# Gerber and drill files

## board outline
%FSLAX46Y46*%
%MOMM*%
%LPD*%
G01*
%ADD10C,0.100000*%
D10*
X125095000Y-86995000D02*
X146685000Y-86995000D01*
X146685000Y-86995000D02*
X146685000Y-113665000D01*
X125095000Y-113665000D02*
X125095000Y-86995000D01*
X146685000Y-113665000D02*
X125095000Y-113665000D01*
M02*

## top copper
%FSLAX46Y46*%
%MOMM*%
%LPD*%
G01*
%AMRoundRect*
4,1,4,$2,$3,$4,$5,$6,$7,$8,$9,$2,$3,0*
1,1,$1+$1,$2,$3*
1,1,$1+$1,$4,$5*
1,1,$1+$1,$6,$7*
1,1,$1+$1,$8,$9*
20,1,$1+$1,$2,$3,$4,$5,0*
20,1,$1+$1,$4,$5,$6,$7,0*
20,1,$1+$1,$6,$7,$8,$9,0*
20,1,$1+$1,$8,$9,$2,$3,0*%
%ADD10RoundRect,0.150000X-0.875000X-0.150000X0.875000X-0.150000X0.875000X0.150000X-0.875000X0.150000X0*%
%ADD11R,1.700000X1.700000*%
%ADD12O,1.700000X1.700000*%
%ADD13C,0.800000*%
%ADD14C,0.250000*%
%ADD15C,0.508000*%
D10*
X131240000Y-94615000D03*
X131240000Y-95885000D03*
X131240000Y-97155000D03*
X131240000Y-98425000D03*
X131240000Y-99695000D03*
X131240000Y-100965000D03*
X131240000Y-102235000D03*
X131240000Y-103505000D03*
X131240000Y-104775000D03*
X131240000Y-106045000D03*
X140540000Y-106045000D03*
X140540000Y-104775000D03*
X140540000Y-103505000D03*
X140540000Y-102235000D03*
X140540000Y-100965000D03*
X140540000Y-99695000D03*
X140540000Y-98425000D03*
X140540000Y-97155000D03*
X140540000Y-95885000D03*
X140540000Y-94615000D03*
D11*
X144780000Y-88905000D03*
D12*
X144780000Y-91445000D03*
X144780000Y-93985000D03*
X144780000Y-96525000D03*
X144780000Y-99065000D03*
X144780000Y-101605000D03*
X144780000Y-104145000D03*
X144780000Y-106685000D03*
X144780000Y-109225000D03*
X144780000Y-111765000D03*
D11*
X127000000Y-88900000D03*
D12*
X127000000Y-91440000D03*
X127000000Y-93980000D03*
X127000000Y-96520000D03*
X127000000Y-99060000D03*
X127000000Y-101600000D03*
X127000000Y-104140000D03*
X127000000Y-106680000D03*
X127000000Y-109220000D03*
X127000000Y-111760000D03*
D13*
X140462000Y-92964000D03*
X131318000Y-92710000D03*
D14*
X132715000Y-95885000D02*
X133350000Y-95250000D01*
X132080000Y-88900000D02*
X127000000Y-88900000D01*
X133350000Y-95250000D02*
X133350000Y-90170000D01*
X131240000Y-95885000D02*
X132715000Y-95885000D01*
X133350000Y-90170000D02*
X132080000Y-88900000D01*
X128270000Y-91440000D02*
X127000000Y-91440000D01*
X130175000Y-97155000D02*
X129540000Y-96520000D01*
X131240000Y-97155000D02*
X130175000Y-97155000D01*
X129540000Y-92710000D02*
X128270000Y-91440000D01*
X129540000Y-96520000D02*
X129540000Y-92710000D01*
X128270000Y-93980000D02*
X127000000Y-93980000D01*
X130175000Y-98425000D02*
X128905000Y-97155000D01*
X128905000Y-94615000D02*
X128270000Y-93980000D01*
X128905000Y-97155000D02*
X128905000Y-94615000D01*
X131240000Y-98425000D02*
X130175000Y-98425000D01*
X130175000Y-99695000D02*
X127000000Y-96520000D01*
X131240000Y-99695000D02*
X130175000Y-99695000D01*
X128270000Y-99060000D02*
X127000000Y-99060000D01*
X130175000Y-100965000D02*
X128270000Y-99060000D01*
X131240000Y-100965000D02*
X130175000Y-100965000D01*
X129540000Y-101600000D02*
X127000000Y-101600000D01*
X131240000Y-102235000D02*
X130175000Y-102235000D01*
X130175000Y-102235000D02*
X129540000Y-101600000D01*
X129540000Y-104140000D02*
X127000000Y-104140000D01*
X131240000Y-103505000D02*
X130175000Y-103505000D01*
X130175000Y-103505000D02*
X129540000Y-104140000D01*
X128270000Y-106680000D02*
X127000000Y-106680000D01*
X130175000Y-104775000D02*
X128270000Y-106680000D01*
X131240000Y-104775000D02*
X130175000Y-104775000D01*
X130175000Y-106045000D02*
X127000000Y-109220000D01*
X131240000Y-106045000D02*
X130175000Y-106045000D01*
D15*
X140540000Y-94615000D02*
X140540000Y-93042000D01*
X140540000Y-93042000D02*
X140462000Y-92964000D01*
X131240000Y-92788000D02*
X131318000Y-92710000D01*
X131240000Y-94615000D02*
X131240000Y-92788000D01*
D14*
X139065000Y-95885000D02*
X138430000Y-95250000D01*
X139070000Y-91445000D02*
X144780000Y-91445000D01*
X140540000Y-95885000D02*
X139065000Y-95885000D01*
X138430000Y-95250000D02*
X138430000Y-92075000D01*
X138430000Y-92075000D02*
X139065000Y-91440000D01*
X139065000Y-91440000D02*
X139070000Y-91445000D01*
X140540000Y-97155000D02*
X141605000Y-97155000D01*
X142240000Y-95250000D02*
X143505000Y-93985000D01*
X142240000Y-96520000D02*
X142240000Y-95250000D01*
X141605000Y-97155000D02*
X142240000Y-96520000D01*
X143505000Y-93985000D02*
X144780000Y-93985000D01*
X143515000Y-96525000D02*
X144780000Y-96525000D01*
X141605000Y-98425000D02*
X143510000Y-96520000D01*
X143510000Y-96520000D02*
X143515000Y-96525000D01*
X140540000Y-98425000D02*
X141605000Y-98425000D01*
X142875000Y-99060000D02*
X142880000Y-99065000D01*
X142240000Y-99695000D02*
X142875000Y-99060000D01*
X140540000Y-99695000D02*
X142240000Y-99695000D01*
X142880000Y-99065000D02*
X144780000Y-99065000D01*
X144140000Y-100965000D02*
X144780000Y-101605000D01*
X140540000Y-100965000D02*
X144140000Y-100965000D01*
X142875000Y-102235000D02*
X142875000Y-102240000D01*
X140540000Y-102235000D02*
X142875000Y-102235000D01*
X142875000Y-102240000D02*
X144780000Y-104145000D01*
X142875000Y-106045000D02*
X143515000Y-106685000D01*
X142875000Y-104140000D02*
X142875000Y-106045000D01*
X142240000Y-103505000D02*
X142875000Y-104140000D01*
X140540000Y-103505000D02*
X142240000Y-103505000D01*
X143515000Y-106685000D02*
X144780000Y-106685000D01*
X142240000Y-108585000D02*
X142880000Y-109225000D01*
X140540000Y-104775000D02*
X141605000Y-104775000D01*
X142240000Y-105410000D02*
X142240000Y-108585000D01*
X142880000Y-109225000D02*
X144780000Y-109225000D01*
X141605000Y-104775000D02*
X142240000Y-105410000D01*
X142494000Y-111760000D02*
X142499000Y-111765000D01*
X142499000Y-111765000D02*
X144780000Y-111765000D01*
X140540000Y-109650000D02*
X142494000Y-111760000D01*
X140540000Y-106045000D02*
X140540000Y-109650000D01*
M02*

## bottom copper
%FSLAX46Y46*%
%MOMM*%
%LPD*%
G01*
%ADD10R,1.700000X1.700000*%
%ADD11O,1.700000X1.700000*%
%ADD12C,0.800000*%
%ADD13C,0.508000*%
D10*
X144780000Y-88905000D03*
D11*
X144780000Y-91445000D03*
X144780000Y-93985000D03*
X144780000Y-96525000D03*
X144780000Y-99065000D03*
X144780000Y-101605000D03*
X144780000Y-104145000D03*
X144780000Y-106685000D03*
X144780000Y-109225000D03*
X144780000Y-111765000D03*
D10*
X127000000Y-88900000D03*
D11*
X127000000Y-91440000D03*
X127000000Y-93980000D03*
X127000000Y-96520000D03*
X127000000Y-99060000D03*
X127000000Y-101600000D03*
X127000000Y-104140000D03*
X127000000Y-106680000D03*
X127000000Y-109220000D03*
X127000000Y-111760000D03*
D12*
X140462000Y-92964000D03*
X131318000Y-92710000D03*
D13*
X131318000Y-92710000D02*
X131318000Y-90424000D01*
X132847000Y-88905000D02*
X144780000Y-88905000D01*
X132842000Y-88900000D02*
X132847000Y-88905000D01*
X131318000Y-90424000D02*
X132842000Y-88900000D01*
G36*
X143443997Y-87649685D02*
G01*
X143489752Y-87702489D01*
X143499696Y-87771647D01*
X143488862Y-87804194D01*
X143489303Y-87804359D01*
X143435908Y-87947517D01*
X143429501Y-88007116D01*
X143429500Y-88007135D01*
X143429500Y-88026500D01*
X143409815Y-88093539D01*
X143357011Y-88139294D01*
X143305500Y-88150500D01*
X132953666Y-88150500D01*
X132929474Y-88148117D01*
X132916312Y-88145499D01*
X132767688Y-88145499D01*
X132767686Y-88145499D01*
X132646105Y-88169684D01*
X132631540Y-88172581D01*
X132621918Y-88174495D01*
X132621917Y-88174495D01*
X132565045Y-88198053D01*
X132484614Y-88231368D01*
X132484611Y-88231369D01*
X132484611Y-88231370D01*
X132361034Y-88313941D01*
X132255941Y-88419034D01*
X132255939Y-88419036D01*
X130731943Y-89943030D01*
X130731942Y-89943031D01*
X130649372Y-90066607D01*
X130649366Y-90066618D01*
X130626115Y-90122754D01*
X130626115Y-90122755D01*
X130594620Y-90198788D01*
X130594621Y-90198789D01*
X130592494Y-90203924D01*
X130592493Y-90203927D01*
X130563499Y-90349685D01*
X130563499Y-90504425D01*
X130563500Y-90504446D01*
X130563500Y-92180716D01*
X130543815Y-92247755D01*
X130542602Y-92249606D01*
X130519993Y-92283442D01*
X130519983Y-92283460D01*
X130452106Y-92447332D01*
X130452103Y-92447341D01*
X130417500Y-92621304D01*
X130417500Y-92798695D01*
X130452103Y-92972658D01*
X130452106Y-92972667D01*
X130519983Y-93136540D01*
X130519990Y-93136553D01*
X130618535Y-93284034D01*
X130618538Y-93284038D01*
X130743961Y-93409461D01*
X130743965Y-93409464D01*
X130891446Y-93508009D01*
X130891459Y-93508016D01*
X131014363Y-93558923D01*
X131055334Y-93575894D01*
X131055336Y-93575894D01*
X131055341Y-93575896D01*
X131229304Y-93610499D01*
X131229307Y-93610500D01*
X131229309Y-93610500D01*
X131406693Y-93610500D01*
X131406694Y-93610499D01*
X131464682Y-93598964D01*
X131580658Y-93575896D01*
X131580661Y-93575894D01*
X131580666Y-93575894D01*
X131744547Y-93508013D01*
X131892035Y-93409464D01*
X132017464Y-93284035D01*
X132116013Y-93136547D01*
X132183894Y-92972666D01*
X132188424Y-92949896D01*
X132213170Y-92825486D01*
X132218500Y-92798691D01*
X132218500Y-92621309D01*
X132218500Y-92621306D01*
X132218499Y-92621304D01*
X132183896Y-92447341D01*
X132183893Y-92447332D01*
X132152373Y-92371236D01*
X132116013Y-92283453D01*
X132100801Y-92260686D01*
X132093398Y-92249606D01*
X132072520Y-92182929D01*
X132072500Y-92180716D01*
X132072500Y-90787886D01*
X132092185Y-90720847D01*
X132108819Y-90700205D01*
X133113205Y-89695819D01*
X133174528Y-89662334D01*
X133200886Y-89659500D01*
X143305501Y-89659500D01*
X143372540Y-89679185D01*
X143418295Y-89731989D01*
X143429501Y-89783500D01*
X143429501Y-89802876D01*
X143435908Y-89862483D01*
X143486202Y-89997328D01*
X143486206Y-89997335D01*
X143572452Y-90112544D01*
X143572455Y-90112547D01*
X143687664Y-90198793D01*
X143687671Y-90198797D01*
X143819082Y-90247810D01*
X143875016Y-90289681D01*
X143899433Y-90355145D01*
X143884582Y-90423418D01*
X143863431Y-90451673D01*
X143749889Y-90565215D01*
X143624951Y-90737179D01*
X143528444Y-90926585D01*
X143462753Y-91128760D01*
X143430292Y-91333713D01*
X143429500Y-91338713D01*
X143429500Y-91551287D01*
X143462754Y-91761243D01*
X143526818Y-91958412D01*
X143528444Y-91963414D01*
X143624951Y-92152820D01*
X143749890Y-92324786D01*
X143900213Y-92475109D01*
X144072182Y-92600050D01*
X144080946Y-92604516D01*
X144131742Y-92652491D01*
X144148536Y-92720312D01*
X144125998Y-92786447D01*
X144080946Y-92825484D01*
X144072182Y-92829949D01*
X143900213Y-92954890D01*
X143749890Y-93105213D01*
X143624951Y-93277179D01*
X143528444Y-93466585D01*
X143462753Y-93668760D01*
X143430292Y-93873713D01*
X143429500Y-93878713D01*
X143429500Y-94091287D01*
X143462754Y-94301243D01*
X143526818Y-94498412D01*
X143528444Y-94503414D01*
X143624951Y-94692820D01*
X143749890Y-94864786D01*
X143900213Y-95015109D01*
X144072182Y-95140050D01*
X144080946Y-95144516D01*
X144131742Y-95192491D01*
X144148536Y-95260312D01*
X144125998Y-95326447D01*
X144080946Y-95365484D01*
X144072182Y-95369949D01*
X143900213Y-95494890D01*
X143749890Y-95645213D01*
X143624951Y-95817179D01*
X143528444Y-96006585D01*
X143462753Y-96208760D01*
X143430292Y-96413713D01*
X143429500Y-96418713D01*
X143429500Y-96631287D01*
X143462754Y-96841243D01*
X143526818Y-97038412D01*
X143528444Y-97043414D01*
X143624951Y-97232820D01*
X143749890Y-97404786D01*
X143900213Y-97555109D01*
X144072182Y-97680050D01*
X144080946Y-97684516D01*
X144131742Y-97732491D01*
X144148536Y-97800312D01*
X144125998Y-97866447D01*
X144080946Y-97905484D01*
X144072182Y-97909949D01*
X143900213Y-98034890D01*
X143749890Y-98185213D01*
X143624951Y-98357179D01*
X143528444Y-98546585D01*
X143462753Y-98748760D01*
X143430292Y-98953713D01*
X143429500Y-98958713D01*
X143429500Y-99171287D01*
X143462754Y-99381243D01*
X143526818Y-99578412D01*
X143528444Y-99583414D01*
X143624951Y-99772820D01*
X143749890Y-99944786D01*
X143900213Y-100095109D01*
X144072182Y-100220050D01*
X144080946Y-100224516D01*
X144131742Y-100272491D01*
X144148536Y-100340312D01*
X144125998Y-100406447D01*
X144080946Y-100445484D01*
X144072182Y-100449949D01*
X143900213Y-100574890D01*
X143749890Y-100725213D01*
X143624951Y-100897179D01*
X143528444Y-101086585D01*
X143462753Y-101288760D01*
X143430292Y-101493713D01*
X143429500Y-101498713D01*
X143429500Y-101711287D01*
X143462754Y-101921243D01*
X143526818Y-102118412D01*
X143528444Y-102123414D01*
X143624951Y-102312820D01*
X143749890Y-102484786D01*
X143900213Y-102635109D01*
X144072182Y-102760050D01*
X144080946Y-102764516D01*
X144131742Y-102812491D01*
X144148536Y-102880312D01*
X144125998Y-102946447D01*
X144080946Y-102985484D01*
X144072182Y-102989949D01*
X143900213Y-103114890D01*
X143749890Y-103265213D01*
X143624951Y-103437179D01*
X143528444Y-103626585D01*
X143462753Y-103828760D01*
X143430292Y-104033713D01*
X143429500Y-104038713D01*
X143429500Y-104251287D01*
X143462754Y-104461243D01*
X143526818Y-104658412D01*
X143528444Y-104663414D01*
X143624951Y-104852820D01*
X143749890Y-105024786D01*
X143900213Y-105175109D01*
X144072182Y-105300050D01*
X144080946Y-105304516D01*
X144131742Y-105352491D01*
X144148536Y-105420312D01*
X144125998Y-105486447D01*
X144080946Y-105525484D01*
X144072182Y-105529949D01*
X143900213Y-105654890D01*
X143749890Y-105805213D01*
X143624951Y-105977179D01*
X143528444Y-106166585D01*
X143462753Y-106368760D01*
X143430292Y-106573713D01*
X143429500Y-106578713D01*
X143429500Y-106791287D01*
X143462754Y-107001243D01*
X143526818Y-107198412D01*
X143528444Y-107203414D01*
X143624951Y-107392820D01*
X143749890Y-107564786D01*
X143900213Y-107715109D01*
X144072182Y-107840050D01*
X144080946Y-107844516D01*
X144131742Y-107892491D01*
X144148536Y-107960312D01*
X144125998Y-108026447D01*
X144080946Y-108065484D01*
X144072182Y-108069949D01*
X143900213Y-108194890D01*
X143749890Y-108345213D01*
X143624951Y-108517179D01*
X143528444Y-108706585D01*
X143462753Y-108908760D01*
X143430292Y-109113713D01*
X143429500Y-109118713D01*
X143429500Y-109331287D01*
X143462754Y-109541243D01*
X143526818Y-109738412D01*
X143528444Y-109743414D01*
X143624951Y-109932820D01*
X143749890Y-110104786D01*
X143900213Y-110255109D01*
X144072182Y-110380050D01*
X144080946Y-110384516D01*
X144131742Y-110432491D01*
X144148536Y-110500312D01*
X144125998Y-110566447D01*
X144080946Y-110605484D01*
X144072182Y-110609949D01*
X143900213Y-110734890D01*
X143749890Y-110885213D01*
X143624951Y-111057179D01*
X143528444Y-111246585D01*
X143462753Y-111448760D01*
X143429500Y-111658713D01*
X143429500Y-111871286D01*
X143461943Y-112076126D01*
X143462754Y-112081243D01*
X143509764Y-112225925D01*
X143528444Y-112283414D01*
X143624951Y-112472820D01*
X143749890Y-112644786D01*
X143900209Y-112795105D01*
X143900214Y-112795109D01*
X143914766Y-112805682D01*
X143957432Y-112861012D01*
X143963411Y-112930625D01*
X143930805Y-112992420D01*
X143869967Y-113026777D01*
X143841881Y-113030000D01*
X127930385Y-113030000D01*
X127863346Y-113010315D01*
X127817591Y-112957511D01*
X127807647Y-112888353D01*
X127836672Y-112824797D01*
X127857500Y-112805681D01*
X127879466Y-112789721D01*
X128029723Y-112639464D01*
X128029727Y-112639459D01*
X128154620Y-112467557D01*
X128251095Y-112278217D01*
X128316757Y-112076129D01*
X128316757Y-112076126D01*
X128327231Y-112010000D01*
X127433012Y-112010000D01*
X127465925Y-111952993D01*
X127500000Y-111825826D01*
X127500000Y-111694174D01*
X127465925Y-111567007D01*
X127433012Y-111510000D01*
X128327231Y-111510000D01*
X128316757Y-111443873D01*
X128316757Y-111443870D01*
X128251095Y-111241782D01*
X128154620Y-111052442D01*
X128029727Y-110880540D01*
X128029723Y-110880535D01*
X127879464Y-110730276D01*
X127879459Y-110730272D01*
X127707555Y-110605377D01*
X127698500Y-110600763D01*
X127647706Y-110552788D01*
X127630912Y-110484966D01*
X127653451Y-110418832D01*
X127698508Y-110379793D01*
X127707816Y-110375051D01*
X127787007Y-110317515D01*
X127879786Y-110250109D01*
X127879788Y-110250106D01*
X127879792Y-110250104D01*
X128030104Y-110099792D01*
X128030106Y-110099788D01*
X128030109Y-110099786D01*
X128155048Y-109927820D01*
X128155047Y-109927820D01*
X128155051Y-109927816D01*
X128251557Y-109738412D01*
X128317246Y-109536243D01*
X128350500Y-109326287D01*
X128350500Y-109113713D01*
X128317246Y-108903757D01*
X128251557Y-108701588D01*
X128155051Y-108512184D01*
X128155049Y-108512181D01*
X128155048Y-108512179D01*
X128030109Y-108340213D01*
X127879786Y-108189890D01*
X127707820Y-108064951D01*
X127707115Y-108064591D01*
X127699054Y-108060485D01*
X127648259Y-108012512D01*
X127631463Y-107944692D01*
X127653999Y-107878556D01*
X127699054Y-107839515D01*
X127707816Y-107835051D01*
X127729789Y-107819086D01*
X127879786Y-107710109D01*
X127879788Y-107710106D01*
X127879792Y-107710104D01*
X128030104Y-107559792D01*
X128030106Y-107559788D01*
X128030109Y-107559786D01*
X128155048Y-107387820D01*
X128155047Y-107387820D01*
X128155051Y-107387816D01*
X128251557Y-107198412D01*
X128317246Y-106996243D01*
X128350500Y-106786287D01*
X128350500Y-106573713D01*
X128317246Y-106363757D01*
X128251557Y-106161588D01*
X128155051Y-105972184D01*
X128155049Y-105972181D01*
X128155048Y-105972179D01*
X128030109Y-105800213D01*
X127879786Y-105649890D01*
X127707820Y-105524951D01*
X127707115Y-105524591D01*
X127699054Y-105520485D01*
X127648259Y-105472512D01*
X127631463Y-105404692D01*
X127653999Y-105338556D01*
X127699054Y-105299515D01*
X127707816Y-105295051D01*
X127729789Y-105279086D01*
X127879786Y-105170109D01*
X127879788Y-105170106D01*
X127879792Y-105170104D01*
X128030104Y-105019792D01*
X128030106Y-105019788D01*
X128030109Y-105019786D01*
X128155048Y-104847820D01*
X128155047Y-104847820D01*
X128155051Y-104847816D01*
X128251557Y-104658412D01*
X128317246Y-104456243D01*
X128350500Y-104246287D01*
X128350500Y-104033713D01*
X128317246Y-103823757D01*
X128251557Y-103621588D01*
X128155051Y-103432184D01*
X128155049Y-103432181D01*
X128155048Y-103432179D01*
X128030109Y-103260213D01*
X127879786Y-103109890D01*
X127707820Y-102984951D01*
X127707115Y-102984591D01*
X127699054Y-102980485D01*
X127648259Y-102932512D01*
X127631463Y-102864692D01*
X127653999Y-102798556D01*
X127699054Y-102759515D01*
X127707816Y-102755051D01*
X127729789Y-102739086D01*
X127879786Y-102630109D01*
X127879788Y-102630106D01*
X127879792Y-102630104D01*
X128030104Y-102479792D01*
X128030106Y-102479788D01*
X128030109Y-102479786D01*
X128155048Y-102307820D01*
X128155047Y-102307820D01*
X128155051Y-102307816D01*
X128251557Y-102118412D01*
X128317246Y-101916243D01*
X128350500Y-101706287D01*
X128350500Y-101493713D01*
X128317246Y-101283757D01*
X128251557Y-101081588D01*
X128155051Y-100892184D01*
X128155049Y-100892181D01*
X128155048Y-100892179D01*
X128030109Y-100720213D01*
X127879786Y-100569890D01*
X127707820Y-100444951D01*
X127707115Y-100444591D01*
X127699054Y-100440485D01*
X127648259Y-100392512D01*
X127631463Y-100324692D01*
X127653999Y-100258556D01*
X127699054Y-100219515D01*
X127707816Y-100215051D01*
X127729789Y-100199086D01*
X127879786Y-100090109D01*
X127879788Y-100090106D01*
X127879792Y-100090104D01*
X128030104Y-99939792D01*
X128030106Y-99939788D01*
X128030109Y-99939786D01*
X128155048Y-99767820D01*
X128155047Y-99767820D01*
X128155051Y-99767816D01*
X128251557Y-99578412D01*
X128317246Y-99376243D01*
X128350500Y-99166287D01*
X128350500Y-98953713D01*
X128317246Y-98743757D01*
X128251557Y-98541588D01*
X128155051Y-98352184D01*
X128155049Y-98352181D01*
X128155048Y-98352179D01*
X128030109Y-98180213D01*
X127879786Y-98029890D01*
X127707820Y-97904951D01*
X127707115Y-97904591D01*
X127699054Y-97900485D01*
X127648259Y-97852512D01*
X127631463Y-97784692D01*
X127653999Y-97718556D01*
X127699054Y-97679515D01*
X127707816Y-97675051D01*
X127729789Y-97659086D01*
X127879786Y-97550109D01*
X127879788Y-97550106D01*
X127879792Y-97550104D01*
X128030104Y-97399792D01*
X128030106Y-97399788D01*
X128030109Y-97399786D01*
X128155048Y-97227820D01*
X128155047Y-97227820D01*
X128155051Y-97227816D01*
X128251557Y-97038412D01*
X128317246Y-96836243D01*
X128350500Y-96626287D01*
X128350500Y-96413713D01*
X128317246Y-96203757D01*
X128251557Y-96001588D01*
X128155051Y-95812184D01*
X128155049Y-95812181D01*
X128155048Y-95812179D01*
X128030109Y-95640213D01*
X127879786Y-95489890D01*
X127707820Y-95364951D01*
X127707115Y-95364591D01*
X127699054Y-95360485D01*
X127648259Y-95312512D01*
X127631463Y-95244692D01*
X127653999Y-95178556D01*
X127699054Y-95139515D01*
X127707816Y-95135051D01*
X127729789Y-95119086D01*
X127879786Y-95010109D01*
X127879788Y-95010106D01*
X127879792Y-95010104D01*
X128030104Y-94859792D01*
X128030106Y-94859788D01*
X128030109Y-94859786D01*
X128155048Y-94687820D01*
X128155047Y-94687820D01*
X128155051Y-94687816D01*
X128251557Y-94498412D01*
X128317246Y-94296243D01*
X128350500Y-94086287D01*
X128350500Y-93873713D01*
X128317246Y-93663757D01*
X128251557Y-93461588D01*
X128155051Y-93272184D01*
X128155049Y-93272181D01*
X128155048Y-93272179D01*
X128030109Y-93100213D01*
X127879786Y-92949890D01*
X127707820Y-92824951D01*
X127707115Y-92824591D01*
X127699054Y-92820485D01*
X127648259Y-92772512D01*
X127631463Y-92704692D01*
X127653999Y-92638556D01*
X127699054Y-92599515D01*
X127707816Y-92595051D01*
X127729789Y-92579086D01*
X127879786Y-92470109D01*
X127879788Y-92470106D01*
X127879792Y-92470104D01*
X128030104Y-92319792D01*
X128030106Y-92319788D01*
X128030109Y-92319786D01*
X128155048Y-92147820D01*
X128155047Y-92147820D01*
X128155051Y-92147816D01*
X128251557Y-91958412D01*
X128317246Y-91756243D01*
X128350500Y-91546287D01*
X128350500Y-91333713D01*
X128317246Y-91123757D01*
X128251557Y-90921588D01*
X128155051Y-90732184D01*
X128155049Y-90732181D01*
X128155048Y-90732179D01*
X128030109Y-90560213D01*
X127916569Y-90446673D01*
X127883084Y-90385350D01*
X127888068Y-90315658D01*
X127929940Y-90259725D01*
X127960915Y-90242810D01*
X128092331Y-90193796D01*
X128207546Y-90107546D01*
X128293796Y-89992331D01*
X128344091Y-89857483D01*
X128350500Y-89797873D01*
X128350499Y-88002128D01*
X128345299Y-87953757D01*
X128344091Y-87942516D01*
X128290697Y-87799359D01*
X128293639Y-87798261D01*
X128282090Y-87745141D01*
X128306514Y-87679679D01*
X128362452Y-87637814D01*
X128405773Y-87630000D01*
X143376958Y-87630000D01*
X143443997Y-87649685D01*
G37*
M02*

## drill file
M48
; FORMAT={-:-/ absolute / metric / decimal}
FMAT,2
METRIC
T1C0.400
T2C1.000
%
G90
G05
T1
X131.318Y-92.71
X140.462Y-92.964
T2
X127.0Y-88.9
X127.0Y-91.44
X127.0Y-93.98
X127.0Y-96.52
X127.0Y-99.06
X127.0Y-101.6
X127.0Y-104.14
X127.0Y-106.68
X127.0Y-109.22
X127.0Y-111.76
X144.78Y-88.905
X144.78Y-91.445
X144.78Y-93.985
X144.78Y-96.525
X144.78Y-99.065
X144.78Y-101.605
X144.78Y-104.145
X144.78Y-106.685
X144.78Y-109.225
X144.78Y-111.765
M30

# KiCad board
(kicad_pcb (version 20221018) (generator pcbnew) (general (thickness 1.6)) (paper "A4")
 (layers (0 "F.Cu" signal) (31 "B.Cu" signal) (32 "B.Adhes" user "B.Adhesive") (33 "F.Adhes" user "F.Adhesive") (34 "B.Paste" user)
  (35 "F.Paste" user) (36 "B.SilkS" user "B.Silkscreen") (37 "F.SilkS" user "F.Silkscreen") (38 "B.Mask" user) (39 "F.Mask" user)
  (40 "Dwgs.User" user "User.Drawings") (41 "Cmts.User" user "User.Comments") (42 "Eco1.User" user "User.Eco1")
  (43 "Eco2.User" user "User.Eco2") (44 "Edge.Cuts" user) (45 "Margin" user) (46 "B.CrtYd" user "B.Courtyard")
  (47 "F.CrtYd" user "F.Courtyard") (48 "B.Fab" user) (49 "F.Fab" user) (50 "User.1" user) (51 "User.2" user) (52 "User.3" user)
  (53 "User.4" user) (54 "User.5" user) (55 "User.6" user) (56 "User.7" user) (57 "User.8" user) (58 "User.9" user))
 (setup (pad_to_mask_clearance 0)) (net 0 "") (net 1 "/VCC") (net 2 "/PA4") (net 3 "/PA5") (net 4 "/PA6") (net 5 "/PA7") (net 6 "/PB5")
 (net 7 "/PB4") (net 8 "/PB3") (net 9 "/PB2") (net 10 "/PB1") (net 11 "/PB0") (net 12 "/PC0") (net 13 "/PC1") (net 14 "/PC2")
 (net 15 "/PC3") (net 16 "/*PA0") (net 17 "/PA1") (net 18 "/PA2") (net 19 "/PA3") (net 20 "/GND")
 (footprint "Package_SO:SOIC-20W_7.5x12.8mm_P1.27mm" (layer "F.Cu") (at 135.89 100.33)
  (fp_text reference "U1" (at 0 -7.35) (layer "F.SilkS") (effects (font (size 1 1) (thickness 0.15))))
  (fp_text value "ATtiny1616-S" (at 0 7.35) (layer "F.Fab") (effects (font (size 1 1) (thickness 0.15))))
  (pad "1" smd roundrect (at -4.65 -5.715) (size 2.05 0.6) (layers "F.Cu" "F.Paste" "F.Mask") (roundrect_rratio 0.25) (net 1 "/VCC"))
  (pad "2" smd roundrect (at -4.65 -4.445) (size 2.05 0.6) (layers "F.Cu" "F.Paste" "F.Mask") (roundrect_rratio 0.25) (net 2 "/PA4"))
  (pad "3" smd roundrect (at -4.65 -3.175) (size 2.05 0.6) (layers "F.Cu" "F.Paste" "F.Mask") (roundrect_rratio 0.25) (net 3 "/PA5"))
  (pad "4" smd roundrect (at -4.65 -1.905) (size 2.05 0.6) (layers "F.Cu" "F.Paste" "F.Mask") (roundrect_rratio 0.25) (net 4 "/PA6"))
  (pad "5" smd roundrect (at -4.65 -0.635) (size 2.05 0.6) (layers "F.Cu" "F.Paste" "F.Mask") (roundrect_rratio 0.25) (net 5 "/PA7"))
  (pad "6" smd roundrect (at -4.65 0.635) (size 2.05 0.6) (layers "F.Cu" "F.Paste" "F.Mask") (roundrect_rratio 0.25) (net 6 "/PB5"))
  (pad "7" smd roundrect (at -4.65 1.905) (size 2.05 0.6) (layers "F.Cu" "F.Paste" "F.Mask") (roundrect_rratio 0.25) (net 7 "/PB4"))
  (pad "8" smd roundrect (at -4.65 3.175) (size 2.05 0.6) (layers "F.Cu" "F.Paste" "F.Mask") (roundrect_rratio 0.25) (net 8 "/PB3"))
  (pad "9" smd roundrect (at -4.65 4.445) (size 2.05 0.6) (layers "F.Cu" "F.Paste" "F.Mask") (roundrect_rratio 0.25) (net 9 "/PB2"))
  (pad "10" smd roundrect (at -4.65 5.715) (size 2.05 0.6) (layers "F.Cu" "F.Paste" "F.Mask") (roundrect_rratio 0.25) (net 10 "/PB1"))
  (pad "11" smd roundrect (at 4.65 5.715) (size 2.05 0.6) (layers "F.Cu" "F.Paste" "F.Mask") (roundrect_rratio 0.25) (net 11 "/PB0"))
  (pad "12" smd roundrect (at 4.65 4.445) (size 2.05 0.6) (layers "F.Cu" "F.Paste" "F.Mask") (roundrect_rratio 0.25) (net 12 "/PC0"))
  (pad "13" smd roundrect (at 4.65 3.175) (size 2.05 0.6) (layers "F.Cu" "F.Paste" "F.Mask") (roundrect_rratio 0.25) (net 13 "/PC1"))
  (pad "14" smd roundrect (at 4.65 1.905) (size 2.05 0.6) (layers "F.Cu" "F.Paste" "F.Mask") (roundrect_rratio 0.25) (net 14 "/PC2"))
  (pad "15" smd roundrect (at 4.65 0.635) (size 2.05 0.6) (layers "F.Cu" "F.Paste" "F.Mask") (roundrect_rratio 0.25) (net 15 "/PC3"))
  (pad "16" smd roundrect (at 4.65 -0.635) (size 2.05 0.6) (layers "F.Cu" "F.Paste" "F.Mask") (roundrect_rratio 0.25) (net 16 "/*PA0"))
  (pad "17" smd roundrect (at 4.65 -1.905) (size 2.05 0.6) (layers "F.Cu" "F.Paste" "F.Mask") (roundrect_rratio 0.25) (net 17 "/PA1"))
  (pad "18" smd roundrect (at 4.65 -3.175) (size 2.05 0.6) (layers "F.Cu" "F.Paste" "F.Mask") (roundrect_rratio 0.25) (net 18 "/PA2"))
  (pad "19" smd roundrect (at 4.65 -4.445) (size 2.05 0.6) (layers "F.Cu" "F.Paste" "F.Mask") (roundrect_rratio 0.25) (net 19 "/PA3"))
  (pad "20" smd roundrect (at 4.65 -5.715) (size 2.05 0.6) (layers "F.Cu" "F.Paste" "F.Mask") (roundrect_rratio 0.25) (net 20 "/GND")))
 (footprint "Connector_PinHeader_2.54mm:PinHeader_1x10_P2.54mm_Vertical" (layer "F.Cu") (at 144.78 88.905)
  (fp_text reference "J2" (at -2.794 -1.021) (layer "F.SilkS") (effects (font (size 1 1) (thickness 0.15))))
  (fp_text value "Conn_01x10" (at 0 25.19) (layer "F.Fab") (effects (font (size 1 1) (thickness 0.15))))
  (pad "1" thru_hole rect (at 0 0) (size 1.7 1.7) (drill 1) (layers "*.Cu" "*.Mask") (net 1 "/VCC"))
  (pad "2" thru_hole oval (at 0 2.54) (size 1.7 1.7) (drill 1) (layers "*.Cu" "*.Mask") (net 19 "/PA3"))
  (pad "3" thru_hole oval (at 0 5.08) (size 1.7 1.7) (drill 1) (layers "*.Cu" "*.Mask") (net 18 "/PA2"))
  (pad "4" thru_hole oval (at 0 7.62) (size 1.7 1.7) (drill 1) (layers "*.Cu" "*.Mask") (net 17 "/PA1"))
  (pad "5" thru_hole oval (at 0 10.16) (size 1.7 1.7) (drill 1) (layers "*.Cu" "*.Mask") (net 16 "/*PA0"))
  (pad "6" thru_hole oval (at 0 12.7) (size 1.7 1.7) (drill 1) (layers "*.Cu" "*.Mask") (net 15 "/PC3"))
  (pad "7" thru_hole oval (at 0 15.24) (size 1.7 1.7) (drill 1) (layers "*.Cu" "*.Mask") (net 14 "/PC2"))
  (pad "8" thru_hole oval (at 0 17.78) (size 1.7 1.7) (drill 1) (layers "*.Cu" "*.Mask") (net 13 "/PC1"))
  (pad "9" thru_hole oval (at 0 20.32) (size 1.7 1.7) (drill 1) (layers "*.Cu" "*.Mask") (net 12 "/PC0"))
  (pad "10" thru_hole oval (at 0 22.86) (size 1.7 1.7) (drill 1) (layers "*.Cu" "*.Mask") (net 11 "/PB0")))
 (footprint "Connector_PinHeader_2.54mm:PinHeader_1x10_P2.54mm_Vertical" (layer "F.Cu") (at 127 88.9)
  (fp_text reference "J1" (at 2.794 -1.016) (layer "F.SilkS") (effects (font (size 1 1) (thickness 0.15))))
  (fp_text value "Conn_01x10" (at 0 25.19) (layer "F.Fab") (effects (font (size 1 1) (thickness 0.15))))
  (pad "1" thru_hole rect (at 0 0) (size 1.7 1.7) (drill 1) (layers "*.Cu" "*.Mask") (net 2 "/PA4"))
  (pad "2" thru_hole oval (at 0 2.54) (size 1.7 1.7) (drill 1) (layers "*.Cu" "*.Mask") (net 3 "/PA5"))
  (pad "3" thru_hole oval (at 0 5.08) (size 1.7 1.7) (drill 1) (layers "*.Cu" "*.Mask") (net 4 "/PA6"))
  (pad "4" thru_hole oval (at 0 7.62) (size 1.7 1.7) (drill 1) (layers "*.Cu" "*.Mask") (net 5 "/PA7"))
  (pad "5" thru_hole oval (at 0 10.16) (size 1.7 1.7) (drill 1) (layers "*.Cu" "*.Mask") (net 6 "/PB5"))
  (pad "6" thru_hole oval (at 0 12.7) (size 1.7 1.7) (drill 1) (layers "*.Cu" "*.Mask") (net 7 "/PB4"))
  (pad "7" thru_hole oval (at 0 15.24) (size 1.7 1.7) (drill 1) (layers "*.Cu" "*.Mask") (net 8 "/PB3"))
  (pad "8" thru_hole oval (at 0 17.78) (size 1.7 1.7) (drill 1) (layers "*.Cu" "*.Mask") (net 9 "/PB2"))
  (pad "9" thru_hole oval (at 0 20.32) (size 1.7 1.7) (drill 1) (layers "*.Cu" "*.Mask") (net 10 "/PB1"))
  (pad "10" thru_hole oval (at 0 22.86) (size 1.7 1.7) (drill 1) (layers "*.Cu" "*.Mask") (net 20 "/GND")))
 (gr_line (start 125.095 86.995) (end 146.685 86.995) (stroke (width 0.1) (type default)) (layer "Edge.Cuts"))
 (gr_line (start 146.685 86.995) (end 146.685 113.665) (stroke (width 0.1) (type default)) (layer "Edge.Cuts"))
 (gr_line (start 125.095 113.665) (end 125.095 86.995) (stroke (width 0.1) (type default)) (layer "Edge.Cuts"))
 (gr_line (start 146.685 113.665) (end 125.095 113.665) (stroke (width 0.1) (type default)) (layer "Edge.Cuts"))
 (segment (start 132.715 95.885) (end 133.35 95.25) (width 0.25) (layer "F.Cu") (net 2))
 (segment (start 132.08 88.9) (end 127 88.9) (width 0.25) (layer "F.Cu") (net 2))
 (segment (start 133.35 95.25) (end 133.35 90.17) (width 0.25) (layer "F.Cu") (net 2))
 (segment (start 131.24 95.885) (end 132.715 95.885) (width 0.25) (layer "F.Cu") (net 2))
 (segment (start 133.35 90.17) (end 132.08 88.9) (width 0.25) (layer "F.Cu") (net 2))
 (segment (start 128.27 91.44) (end 127 91.44) (width 0.25) (layer "F.Cu") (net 3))
 (segment (start 130.175 97.155) (end 129.54 96.52) (width 0.25) (layer "F.Cu") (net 3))
 (segment (start 131.24 97.155) (end 130.175 97.155) (width 0.25) (layer "F.Cu") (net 3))
 (segment (start 129.54 92.71) (end 128.27 91.44) (width 0.25) (layer "F.Cu") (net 3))
 (segment (start 129.54 96.52) (end 129.54 92.71) (width 0.25) (layer "F.Cu") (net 3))
 (segment (start 128.27 93.98) (end 127 93.98) (width 0.25) (layer "F.Cu") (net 4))
 (segment (start 130.175 98.425) (end 128.905 97.155) (width 0.25) (layer "F.Cu") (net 4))
 (segment (start 128.905 94.615) (end 128.27 93.98) (width 0.25) (layer "F.Cu") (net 4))
 (segment (start 128.905 97.155) (end 128.905 94.615) (width 0.25) (layer "F.Cu") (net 4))
 (segment (start 131.24 98.425) (end 130.175 98.425) (width 0.25) (layer "F.Cu") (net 4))
 (segment (start 130.175 99.695) (end 127 96.52) (width 0.25) (layer "F.Cu") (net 5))
 (segment (start 131.24 99.695) (end 130.175 99.695) (width 0.25) (layer "F.Cu") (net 5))
 (segment (start 128.27 99.06) (end 127 99.06) (width 0.25) (layer "F.Cu") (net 6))
 (segment (start 130.175 100.965) (end 128.27 99.06) (width 0.25) (layer "F.Cu") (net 6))
 (segment (start 131.24 100.965) (end 130.175 100.965) (width 0.25) (layer "F.Cu") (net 6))
 (segment (start 129.54 101.6) (end 127 101.6) (width 0.25) (layer "F.Cu") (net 7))
 (segment (start 131.24 102.235) (end 130.175 102.235) (width 0.25) (layer "F.Cu") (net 7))
 (segment (start 130.175 102.235) (end 129.54 101.6) (width 0.25) (layer "F.Cu") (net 7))
 (segment (start 129.54 104.14) (end 127 104.14) (width 0.25) (layer "F.Cu") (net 8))
 (segment (start 131.24 103.505) (end 130.175 103.505) (width 0.25) (layer "F.Cu") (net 8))
 (segment (start 130.175 103.505) (end 129.54 104.14) (width 0.25) (layer "F.Cu") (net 8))
 (segment (start 128.27 106.68) (end 127 106.68) (width 0.25) (layer "F.Cu") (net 9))
 (segment (start 130.175 104.775) (end 128.27 106.68) (width 0.25) (layer "F.Cu") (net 9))
 (segment (start 131.24 104.775) (end 130.175 104.775) (width 0.25) (layer "F.Cu") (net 9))
 (segment (start 130.175 106.045) (end 127 109.22) (width 0.25) (layer "F.Cu") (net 10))
 (segment (start 131.24 106.045) (end 130.175 106.045) (width 0.25) (layer "F.Cu") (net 10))
 (segment (start 140.54 94.615) (end 140.54 93.042) (width 0.508) (layer "F.Cu") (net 20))
 (segment (start 140.54 93.042) (end 140.462 92.964) (width 0.508) (layer "F.Cu") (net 20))
 (via (at 140.462 92.964) (size 0.8) (drill 0.4) (layers "F.Cu" "B.Cu") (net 20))
 (segment (start 131.24 92.788) (end 131.318 92.71) (width 0.508) (layer "F.Cu") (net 1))
 (segment (start 131.24 94.615) (end 131.24 92.788) (width 0.508) (layer "F.Cu") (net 1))
 (via (at 131.318 92.71) (size 0.8) (drill 0.4) (layers "F.Cu" "B.Cu") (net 1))
 (segment (start 131.318 92.71) (end 131.318 90.424) (width 0.508) (layer "B.Cu") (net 1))
 (segment (start 132.847 88.905) (end 144.78 88.905) (width 0.508) (layer "B.Cu") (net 1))
 (segment (start 132.842 88.9) (end 132.847 88.905) (width 0.508) (layer "B.Cu") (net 1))
 (segment (start 131.318 90.424) (end 132.842 88.9) (width 0.508) (layer "B.Cu") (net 1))
 (segment (start 139.065 95.885) (end 138.43 95.25) (width 0.25) (layer "F.Cu") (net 19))
 (segment (start 139.07 91.445) (end 144.78 91.445) (width 0.25) (layer "F.Cu") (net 19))
 (segment (start 140.54 95.885) (end 139.065 95.885) (width 0.25) (layer "F.Cu") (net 19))
 (segment (start 138.43 95.25) (end 138.43 92.075) (width 0.25) (layer "F.Cu") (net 19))
 (segment (start 138.43 92.075) (end 139.065 91.44) (width 0.25) (layer "F.Cu") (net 19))
 (segment (start 139.065 91.44) (end 139.07 91.445) (width 0.25) (layer "F.Cu") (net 19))
 (segment (start 140.54 97.155) (end 141.605 97.155) (width 0.25) (layer "F.Cu") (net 18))
 (segment (start 142.24 95.25) (end 143.505 93.985) (width 0.25) (layer "F.Cu") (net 18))
 (segment (start 142.24 96.52) (end 142.24 95.25) (width 0.25) (layer "F.Cu") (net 18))
 (segment (start 141.605 97.155) (end 142.24 96.52) (width 0.25) (layer "F.Cu") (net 18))
 (segment (start 143.505 93.985) (end 144.78 93.985) (width 0.25) (layer "F.Cu") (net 18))
 (segment (start 143.515 96.525) (end 144.78 96.525) (width 0.25) (layer "F.Cu") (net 17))
 (segment (start 141.605 98.425) (end 143.51 96.52) (width 0.25) (layer "F.Cu") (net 17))
 (segment (start 143.51 96.52) (end 143.515 96.525) (width 0.25) (layer "F.Cu") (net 17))
 (segment (start 140.54 98.425) (end 141.605 98.425) (width 0.25) (layer "F.Cu") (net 17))
 (segment (start 142.875 99.06) (end 142.88 99.065) (width 0.25) (layer "F.Cu") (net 16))
 (segment (start 142.24 99.695) (end 142.875 99.06) (width 0.25) (layer "F.Cu") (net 16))
 (segment (start 140.54 99.695) (end 142.24 99.695) (width 0.25) (layer "F.Cu") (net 16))
 (segment (start 142.88 99.065) (end 144.78 99.065) (width 0.25) (layer "F.Cu") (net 16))
 (segment (start 144.14 100.965) (end 144.78 101.605) (width 0.25) (layer "F.Cu") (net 15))
 (segment (start 140.54 100.965) (end 144.14 100.965) (width 0.25) (layer "F.Cu") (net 15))
 (segment (start 142.875 102.235) (end 142.875 102.24) (width 0.25) (layer "F.Cu") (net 14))
 (segment (start 140.54 102.235) (end 142.875 102.235) (width 0.25) (layer "F.Cu") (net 14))
 (segment (start 142.875 102.24) (end 144.78 104.145) (width 0.25) (layer "F.Cu") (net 14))
 (segment (start 142.875 106.045) (end 143.515 106.685) (width 0.25) (layer "F.Cu") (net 13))
 (segment (start 142.875 104.14) (end 142.875 106.045) (width 0.25) (layer "F.Cu") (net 13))
 (segment (start 142.24 103.505) (end 142.875 104.14) (width 0.25) (layer "F.Cu") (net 13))
 (segment (start 140.54 103.505) (end 142.24 103.505) (width 0.25) (layer "F.Cu") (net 13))
 (segment (start 143.515 106.685) (end 144.78 106.685) (width 0.25) (layer "F.Cu") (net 13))
 (segment (start 142.24 108.585) (end 142.88 109.225) (width 0.25) (layer "F.Cu") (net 12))
 (segment (start 140.54 104.775) (end 141.605 104.775) (width 0.25) (layer "F.Cu") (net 12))
 (segment (start 142.24 105.41) (end 142.24 108.585) (width 0.25) (layer "F.Cu") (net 12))
 (segment (start 142.88 109.225) (end 144.78 109.225) (width 0.25) (layer "F.Cu") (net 12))
 (segment (start 141.605 104.775) (end 142.24 105.41) (width 0.25) (layer "F.Cu") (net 12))
 (segment (start 142.494 111.76) (end 142.499 111.765) (width 0.25) (layer "F.Cu") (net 11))
 (segment (start 142.499 111.765) (end 144.78 111.765) (width 0.25) (layer "F.Cu") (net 11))
 (segment (start 140.54 109.65) (end 142.494 111.76) (width 0.25) (layer "F.Cu") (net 11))
 (segment (start 140.54 106.045) (end 140.54 109.65) (width 0.25) (layer "F.Cu") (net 11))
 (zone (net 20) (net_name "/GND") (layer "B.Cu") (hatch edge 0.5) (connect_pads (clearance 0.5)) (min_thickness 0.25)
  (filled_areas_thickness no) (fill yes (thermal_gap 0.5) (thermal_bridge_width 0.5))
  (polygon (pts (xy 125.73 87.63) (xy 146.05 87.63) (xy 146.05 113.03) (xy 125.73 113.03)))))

